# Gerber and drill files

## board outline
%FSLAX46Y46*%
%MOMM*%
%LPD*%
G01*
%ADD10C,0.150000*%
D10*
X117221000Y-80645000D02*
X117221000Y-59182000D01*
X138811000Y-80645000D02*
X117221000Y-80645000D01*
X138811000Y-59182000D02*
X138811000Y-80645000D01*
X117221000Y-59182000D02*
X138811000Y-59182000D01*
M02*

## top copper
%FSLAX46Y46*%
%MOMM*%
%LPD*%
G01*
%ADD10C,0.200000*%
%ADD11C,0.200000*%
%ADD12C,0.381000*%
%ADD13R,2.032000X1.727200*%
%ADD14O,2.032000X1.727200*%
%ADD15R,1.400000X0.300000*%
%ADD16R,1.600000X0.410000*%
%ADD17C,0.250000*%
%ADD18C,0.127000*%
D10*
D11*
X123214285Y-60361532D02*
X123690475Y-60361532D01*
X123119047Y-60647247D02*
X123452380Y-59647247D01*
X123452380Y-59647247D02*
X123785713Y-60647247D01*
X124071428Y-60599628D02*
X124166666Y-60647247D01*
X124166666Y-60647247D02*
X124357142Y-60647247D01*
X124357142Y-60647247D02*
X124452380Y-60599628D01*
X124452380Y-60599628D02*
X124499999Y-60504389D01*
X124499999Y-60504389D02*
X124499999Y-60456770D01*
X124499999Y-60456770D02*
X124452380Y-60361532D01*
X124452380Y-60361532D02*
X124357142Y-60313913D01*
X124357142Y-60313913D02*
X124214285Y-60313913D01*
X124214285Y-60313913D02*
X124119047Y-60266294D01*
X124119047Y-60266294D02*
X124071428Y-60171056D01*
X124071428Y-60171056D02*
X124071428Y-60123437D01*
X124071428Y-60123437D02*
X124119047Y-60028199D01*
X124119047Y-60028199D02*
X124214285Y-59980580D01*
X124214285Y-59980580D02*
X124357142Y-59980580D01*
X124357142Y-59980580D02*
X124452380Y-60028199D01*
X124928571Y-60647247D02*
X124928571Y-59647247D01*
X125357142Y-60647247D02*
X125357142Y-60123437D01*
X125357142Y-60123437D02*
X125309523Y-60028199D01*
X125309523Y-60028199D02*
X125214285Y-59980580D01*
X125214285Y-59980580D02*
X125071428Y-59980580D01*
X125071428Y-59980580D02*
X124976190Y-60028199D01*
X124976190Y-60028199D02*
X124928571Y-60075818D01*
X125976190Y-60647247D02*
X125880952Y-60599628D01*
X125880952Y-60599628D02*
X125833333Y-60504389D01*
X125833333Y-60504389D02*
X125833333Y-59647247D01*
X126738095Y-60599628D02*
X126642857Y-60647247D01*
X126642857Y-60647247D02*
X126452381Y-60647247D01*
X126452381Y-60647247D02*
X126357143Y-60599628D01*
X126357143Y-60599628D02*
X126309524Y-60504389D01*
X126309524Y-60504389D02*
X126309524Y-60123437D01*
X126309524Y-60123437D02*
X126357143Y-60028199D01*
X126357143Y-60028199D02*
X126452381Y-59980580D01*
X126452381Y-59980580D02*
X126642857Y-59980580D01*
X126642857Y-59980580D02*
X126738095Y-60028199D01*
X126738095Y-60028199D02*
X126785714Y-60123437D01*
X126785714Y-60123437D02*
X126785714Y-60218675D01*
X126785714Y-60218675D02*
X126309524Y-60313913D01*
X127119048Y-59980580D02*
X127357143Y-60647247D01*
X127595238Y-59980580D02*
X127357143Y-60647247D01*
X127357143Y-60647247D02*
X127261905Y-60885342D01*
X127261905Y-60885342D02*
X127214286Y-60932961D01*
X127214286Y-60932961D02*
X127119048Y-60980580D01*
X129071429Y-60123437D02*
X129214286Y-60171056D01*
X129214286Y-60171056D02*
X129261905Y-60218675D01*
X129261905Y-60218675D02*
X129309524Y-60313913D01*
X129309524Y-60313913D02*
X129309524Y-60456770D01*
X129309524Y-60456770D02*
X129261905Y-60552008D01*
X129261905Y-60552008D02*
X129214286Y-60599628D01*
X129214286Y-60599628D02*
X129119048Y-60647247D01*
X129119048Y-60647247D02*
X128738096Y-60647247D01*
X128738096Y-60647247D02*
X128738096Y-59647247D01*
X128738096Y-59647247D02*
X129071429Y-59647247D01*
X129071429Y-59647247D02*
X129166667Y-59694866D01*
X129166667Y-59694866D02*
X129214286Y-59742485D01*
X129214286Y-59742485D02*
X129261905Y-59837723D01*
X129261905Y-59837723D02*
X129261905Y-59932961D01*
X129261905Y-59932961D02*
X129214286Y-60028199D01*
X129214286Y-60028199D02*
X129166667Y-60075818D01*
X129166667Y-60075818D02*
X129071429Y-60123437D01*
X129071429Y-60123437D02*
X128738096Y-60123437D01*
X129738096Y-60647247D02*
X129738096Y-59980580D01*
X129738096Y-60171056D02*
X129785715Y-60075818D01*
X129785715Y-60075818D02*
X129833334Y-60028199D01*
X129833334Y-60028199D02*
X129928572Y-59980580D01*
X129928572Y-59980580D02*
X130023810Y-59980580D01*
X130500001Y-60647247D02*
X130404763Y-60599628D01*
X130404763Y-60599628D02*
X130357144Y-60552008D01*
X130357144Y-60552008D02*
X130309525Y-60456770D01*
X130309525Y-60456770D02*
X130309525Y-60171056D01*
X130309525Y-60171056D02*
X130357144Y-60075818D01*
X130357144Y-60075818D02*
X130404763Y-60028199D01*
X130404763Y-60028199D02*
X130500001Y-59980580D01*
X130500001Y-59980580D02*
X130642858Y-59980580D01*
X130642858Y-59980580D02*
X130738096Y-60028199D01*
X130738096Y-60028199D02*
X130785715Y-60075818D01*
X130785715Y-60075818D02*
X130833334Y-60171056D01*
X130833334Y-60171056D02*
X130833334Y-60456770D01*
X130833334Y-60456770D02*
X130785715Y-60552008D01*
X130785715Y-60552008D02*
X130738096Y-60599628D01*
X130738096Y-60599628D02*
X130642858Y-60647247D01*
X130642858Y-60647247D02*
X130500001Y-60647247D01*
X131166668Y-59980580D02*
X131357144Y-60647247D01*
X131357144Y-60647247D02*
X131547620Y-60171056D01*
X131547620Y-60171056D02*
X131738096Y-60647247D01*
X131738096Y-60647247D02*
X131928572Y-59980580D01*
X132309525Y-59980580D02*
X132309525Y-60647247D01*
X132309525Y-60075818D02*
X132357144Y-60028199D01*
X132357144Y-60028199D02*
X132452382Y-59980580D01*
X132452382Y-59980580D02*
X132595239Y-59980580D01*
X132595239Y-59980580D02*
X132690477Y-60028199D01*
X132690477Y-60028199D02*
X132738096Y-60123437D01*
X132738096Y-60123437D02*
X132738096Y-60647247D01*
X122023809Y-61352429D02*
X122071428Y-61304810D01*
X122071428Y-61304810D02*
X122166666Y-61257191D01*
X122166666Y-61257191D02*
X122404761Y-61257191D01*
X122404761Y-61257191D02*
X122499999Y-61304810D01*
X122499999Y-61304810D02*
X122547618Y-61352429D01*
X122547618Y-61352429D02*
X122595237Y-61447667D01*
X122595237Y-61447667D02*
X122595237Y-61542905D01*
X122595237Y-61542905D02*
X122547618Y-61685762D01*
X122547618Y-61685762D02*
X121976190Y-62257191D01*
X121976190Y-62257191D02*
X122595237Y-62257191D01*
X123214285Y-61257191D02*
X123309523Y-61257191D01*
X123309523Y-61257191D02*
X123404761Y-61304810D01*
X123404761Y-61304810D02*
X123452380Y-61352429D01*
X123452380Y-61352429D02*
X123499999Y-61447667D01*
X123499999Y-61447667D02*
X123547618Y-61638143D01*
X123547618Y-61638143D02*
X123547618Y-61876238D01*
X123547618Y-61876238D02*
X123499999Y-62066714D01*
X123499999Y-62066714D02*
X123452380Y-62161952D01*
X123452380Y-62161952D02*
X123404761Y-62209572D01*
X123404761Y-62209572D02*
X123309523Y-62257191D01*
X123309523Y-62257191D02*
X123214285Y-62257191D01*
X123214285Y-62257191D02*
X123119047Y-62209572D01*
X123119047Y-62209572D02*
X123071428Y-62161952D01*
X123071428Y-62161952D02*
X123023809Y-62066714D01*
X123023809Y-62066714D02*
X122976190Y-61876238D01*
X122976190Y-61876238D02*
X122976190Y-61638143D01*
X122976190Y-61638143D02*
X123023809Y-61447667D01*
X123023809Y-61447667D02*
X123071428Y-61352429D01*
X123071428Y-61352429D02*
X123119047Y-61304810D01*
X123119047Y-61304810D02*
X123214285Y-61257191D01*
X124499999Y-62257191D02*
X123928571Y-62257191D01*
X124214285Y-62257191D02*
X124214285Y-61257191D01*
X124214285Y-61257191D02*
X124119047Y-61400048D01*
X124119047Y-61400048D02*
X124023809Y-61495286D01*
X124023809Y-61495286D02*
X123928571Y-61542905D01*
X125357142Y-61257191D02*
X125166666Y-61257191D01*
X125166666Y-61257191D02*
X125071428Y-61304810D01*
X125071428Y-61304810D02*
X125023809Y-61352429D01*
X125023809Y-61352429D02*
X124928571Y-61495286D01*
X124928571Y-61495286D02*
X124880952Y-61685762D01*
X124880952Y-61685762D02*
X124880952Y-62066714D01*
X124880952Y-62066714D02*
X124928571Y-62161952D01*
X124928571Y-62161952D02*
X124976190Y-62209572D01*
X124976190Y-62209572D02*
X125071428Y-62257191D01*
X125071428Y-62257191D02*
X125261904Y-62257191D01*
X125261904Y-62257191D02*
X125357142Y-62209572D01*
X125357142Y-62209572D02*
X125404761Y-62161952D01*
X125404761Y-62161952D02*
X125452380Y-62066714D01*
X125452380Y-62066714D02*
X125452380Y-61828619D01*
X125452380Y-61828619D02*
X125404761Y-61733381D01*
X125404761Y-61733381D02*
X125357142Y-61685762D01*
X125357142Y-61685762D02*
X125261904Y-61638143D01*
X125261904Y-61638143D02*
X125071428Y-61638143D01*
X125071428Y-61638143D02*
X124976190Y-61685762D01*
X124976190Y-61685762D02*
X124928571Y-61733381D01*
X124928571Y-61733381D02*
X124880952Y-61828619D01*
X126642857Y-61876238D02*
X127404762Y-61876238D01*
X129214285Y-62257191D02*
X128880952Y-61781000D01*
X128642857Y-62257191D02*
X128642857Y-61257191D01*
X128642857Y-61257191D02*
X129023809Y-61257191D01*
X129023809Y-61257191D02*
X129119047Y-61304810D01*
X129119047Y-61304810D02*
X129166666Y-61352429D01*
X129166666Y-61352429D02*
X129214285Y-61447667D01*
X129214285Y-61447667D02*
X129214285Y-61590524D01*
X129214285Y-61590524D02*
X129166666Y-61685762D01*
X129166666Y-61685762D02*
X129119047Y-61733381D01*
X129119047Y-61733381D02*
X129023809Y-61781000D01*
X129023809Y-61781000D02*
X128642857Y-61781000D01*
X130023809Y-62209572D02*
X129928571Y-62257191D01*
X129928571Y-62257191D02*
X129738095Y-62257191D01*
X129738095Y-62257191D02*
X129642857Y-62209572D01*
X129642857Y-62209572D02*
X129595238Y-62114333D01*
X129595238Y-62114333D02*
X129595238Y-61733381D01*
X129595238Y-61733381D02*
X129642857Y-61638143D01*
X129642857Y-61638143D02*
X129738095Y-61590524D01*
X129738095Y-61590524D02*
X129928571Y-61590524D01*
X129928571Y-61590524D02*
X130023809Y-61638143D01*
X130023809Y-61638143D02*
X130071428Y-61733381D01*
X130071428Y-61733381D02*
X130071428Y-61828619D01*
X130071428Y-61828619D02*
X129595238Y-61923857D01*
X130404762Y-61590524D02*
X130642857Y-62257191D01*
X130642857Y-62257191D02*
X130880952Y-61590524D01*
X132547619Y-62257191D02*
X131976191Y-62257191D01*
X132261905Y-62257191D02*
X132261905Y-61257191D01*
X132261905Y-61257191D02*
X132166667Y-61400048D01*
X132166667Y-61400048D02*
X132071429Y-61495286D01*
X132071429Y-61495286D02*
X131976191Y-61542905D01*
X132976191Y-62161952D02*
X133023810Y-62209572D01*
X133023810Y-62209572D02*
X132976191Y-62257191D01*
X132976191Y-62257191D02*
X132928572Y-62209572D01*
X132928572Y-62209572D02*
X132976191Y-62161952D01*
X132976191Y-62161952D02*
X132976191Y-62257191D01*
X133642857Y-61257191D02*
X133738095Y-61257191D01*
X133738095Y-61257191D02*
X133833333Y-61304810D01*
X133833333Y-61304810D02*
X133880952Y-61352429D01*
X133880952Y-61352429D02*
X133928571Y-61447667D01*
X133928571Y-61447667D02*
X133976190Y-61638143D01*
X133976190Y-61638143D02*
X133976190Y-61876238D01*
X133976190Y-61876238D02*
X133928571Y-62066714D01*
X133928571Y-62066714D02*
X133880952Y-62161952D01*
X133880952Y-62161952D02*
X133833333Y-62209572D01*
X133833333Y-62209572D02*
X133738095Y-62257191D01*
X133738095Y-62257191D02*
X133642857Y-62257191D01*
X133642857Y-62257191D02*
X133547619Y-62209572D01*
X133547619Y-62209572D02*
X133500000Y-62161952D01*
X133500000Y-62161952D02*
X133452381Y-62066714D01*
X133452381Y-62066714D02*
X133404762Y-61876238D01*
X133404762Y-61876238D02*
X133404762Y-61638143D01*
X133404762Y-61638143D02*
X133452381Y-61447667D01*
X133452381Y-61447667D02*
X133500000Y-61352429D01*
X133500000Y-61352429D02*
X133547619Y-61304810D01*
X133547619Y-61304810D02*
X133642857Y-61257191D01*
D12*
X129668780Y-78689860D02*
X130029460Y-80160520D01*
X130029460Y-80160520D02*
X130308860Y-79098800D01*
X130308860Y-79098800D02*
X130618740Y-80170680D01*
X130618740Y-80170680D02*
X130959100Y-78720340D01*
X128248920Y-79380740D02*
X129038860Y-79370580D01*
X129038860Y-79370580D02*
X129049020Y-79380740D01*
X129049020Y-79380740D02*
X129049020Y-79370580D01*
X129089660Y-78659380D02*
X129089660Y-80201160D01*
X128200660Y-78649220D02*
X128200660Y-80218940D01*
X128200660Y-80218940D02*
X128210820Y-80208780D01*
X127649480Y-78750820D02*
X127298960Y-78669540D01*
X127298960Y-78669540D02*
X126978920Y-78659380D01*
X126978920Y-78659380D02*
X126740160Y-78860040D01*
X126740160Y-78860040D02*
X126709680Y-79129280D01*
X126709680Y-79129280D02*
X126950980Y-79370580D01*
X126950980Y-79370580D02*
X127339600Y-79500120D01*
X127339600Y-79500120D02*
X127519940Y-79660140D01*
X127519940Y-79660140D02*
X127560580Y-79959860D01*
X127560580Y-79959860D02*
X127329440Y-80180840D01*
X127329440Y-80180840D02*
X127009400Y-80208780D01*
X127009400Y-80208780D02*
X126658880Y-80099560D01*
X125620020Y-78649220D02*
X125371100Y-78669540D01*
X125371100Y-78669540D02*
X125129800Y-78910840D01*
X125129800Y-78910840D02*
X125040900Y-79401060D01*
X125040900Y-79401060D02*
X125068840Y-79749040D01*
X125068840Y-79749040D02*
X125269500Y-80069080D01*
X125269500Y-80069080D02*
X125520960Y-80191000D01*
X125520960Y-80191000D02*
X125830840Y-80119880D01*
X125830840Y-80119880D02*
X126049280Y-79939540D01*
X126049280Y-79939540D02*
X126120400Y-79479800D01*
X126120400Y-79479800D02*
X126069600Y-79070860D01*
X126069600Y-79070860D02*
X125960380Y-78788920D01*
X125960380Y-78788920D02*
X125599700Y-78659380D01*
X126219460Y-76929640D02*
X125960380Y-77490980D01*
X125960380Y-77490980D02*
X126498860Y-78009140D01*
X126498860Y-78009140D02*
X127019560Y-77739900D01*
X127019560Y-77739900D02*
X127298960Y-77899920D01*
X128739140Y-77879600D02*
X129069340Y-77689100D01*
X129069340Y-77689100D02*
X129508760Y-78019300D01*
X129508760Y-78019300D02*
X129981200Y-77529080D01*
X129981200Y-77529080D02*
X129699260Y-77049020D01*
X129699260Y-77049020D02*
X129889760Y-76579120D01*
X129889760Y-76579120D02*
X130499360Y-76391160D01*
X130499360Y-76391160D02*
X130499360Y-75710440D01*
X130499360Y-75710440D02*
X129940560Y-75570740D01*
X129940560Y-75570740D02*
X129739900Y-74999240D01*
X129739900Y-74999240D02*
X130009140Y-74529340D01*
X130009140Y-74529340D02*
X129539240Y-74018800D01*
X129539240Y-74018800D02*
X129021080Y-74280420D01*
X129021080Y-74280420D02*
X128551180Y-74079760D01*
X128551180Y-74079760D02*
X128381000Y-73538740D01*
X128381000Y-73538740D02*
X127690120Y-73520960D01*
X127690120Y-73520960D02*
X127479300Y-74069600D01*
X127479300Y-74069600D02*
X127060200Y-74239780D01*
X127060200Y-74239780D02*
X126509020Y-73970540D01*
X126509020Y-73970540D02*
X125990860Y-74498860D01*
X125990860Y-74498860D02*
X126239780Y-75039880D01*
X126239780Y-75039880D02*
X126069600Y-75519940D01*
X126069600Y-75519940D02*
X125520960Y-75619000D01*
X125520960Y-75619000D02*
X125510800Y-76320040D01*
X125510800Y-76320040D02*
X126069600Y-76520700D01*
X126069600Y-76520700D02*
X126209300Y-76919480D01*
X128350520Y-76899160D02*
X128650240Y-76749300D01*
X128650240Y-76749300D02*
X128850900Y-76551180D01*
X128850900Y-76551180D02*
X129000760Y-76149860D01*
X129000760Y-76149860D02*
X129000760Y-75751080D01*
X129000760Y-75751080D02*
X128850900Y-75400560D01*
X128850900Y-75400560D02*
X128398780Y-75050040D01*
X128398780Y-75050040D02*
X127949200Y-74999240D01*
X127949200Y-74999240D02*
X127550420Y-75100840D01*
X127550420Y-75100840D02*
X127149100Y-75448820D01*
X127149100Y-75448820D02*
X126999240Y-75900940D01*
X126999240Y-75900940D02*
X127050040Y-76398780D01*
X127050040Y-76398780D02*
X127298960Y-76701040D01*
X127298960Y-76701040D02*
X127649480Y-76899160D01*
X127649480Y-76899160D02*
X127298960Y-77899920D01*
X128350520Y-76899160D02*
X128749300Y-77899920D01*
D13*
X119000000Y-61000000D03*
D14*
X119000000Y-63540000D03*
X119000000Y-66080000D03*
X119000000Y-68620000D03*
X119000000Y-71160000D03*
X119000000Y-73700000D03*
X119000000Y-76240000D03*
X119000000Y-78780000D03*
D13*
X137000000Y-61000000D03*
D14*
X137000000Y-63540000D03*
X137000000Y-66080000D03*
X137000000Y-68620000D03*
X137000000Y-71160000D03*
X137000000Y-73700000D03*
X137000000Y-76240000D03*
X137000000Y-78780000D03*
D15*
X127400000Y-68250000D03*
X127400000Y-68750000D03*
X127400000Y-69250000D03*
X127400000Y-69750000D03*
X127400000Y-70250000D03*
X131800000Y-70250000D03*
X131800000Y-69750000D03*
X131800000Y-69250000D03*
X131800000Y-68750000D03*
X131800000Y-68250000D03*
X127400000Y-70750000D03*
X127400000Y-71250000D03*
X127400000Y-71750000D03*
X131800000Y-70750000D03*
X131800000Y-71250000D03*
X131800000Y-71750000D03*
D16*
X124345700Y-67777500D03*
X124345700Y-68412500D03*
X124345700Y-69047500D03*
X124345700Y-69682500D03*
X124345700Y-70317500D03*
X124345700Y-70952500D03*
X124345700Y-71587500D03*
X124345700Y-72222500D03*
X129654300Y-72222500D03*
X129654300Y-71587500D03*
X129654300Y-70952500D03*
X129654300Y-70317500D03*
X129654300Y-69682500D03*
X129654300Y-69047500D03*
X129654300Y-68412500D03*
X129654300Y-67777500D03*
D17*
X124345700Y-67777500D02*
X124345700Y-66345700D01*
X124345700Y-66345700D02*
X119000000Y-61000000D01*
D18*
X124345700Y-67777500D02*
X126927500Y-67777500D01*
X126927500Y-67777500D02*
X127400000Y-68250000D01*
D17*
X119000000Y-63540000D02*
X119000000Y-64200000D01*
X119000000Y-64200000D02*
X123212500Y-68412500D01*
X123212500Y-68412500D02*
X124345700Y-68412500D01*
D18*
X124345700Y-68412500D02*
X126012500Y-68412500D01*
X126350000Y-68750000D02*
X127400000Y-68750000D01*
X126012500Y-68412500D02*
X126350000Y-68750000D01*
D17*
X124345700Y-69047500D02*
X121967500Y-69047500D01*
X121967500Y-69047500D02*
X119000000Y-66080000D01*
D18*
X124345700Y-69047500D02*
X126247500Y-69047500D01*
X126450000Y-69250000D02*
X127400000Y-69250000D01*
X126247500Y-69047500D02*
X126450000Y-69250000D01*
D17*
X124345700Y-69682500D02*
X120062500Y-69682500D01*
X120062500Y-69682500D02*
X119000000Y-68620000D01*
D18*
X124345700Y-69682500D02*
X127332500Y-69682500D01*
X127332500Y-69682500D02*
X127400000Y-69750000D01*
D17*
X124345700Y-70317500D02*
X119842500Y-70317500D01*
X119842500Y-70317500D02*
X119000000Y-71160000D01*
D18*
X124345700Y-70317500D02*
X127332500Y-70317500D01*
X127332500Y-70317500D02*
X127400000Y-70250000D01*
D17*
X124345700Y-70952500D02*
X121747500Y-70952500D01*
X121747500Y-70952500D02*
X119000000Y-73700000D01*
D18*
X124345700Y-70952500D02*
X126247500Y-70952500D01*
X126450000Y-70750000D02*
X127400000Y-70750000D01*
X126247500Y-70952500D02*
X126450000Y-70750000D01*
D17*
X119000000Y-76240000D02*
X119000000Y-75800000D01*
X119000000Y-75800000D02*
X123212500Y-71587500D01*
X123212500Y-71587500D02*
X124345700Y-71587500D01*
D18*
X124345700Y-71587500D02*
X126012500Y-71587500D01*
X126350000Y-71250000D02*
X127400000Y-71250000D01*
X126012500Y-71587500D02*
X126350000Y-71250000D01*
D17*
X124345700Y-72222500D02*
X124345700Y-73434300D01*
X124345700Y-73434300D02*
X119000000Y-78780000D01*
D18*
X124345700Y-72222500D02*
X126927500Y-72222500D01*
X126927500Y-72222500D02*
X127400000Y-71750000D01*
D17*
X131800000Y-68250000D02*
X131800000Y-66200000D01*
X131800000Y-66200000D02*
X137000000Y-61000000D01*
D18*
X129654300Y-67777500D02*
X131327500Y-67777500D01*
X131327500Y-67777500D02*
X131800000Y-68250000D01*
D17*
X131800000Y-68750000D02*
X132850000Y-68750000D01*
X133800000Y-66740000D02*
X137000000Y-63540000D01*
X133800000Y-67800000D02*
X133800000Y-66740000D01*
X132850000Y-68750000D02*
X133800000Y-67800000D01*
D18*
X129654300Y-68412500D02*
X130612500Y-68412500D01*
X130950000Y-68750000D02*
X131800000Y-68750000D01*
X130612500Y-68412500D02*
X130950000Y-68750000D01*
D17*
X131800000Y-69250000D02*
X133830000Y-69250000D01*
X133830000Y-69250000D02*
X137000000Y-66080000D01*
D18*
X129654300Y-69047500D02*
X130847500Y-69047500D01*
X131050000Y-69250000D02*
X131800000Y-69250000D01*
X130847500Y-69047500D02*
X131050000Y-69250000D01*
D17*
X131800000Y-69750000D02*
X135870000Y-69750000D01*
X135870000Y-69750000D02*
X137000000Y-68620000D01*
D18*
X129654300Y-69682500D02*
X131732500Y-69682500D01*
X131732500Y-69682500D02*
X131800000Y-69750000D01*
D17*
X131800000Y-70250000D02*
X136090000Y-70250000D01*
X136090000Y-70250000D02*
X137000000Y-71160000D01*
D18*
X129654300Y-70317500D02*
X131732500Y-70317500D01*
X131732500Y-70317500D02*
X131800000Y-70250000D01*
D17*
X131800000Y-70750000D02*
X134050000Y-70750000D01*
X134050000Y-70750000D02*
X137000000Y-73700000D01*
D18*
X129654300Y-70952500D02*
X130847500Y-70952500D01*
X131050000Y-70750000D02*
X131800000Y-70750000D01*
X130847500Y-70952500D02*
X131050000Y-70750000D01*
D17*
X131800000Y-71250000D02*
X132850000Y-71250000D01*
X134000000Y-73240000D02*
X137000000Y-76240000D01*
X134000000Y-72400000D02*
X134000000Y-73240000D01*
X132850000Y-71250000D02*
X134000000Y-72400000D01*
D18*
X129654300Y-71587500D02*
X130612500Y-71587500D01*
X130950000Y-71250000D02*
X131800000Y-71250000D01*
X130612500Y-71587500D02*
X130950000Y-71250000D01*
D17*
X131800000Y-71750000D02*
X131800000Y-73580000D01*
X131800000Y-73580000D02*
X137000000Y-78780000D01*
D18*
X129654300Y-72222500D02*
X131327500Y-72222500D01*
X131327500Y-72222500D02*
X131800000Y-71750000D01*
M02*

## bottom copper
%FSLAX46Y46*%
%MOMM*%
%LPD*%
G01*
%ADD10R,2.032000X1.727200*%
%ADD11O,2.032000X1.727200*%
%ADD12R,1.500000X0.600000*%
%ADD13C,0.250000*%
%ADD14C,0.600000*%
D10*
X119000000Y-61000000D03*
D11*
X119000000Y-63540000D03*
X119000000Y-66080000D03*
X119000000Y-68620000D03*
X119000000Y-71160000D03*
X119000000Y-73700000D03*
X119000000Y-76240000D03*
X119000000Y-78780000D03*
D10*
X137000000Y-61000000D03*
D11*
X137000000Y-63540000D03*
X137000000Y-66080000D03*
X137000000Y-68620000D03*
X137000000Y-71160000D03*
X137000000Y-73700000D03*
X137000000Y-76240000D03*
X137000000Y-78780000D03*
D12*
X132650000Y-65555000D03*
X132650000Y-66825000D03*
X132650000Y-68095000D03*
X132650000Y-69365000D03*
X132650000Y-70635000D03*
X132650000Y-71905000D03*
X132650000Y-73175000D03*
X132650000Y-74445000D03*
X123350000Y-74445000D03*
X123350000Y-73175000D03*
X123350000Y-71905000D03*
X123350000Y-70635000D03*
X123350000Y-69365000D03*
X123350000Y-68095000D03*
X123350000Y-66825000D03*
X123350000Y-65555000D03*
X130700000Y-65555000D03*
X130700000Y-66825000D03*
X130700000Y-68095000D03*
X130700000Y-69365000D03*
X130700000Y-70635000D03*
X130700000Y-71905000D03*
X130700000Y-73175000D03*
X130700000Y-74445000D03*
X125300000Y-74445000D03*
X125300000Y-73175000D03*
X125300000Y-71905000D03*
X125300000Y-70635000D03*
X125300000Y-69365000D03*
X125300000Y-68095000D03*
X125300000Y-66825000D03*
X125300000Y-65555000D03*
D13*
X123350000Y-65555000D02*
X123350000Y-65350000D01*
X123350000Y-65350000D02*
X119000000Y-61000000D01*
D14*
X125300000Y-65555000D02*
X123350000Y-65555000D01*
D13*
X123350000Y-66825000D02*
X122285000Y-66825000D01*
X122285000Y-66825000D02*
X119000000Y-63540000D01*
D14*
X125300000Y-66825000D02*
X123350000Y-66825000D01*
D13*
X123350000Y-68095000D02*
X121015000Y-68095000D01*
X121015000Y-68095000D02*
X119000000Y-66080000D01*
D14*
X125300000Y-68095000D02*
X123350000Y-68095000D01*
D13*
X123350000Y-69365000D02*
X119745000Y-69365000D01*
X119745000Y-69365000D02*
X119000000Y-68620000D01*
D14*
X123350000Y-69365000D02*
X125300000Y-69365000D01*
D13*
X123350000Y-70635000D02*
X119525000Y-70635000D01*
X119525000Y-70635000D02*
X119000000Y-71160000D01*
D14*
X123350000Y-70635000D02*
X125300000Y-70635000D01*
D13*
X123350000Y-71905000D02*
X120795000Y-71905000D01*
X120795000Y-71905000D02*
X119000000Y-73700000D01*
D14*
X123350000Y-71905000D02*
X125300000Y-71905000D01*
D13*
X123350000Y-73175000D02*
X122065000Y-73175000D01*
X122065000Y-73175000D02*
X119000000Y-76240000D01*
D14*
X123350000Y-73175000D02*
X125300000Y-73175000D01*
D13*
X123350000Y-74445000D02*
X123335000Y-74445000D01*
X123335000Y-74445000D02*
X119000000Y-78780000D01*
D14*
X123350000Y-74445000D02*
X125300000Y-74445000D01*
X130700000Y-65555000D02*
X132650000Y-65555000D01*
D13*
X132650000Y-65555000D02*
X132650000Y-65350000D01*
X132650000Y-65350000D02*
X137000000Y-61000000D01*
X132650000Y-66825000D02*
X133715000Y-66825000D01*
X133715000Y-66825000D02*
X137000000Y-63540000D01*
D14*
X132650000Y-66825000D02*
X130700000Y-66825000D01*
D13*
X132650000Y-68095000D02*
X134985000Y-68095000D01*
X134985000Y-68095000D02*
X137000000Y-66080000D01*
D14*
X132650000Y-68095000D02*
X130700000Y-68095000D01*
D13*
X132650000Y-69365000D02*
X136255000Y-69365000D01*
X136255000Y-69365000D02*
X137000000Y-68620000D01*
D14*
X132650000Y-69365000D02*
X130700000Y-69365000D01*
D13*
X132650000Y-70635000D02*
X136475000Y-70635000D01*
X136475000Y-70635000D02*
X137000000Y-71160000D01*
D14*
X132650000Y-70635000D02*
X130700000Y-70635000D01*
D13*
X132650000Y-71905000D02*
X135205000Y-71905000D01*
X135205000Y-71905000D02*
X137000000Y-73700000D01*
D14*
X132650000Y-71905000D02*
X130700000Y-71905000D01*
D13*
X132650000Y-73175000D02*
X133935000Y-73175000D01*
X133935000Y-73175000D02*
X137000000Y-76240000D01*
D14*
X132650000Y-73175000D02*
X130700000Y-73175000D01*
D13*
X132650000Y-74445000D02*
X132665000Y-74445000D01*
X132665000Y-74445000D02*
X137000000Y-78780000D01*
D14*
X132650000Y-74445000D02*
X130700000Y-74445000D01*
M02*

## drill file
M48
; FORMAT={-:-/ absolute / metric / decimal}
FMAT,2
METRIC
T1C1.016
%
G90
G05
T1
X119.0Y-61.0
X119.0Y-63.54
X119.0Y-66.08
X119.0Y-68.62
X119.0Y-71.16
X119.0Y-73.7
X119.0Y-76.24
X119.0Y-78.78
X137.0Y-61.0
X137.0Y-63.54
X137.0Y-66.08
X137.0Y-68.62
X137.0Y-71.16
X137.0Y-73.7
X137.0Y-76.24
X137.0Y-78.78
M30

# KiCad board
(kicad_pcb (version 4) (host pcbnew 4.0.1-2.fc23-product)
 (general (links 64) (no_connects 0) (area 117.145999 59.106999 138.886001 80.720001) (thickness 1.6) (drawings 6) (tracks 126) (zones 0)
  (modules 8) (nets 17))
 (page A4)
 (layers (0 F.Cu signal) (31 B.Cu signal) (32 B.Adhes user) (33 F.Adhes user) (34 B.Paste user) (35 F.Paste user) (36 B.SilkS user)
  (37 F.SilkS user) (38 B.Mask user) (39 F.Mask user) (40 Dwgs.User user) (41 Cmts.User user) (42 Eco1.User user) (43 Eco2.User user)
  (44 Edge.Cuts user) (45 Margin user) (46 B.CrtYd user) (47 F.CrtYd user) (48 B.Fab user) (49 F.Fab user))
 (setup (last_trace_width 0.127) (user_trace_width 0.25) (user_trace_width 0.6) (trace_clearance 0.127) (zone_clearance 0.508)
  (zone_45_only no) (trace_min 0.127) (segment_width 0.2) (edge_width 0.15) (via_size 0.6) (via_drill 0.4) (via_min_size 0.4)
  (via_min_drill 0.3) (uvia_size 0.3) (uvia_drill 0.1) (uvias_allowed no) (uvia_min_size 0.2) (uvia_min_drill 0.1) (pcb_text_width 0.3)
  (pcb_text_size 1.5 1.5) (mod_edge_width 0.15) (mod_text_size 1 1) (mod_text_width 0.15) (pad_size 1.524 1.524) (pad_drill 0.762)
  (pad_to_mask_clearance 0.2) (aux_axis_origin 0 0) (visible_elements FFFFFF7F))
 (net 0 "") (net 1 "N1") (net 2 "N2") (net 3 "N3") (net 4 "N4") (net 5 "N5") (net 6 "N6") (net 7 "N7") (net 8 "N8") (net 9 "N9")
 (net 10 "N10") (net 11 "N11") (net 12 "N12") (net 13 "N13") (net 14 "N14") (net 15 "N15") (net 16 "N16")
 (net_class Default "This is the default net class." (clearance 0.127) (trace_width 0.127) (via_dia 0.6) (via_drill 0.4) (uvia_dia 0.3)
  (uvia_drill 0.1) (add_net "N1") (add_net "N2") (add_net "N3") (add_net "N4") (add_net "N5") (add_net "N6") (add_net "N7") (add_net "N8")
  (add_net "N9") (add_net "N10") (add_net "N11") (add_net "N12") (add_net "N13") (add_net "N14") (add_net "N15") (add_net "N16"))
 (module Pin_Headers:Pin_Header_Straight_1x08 (layer F.Cu) (at 119 61)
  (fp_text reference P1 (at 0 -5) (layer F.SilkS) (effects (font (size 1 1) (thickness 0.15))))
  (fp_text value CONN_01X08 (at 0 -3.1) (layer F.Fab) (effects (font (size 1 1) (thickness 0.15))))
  (pad 1 thru_hole rect (at 0 0) (size 2.032 1.7272) (drill 1.016) (layers *.Cu *.Mask F.SilkS) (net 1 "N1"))
  (pad 2 thru_hole oval (at 0 2.54) (size 2.032 1.7272) (drill 1.016) (layers *.Cu *.Mask F.SilkS) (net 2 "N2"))
  (pad 3 thru_hole oval (at 0 5.08) (size 2.032 1.7272) (drill 1.016) (layers *.Cu *.Mask F.SilkS) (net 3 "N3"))
  (pad 4 thru_hole oval (at 0 7.62) (size 2.032 1.7272) (drill 1.016) (layers *.Cu *.Mask F.SilkS) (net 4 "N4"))
  (pad 5 thru_hole oval (at 0 10.16) (size 2.032 1.7272) (drill 1.016) (layers *.Cu *.Mask F.SilkS) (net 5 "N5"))
  (pad 6 thru_hole oval (at 0 12.7) (size 2.032 1.7272) (drill 1.016) (layers *.Cu *.Mask F.SilkS) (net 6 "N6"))
  (pad 7 thru_hole oval (at 0 15.24) (size 2.032 1.7272) (drill 1.016) (layers *.Cu *.Mask F.SilkS) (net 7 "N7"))
  (pad 8 thru_hole oval (at 0 17.78) (size 2.032 1.7272) (drill 1.016) (layers *.Cu *.Mask F.SilkS) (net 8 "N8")))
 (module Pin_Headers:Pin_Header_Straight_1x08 (layer F.Cu) (at 137 61)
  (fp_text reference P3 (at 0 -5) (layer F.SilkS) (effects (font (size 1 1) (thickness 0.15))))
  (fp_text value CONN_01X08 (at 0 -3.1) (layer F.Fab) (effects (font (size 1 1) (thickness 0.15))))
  (pad 1 thru_hole rect (at 0 0) (size 2.032 1.7272) (drill 1.016) (layers *.Cu *.Mask F.SilkS) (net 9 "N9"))
  (pad 2 thru_hole oval (at 0 2.54) (size 2.032 1.7272) (drill 1.016) (layers *.Cu *.Mask F.SilkS) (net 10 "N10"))
  (pad 3 thru_hole oval (at 0 5.08) (size 2.032 1.7272) (drill 1.016) (layers *.Cu *.Mask F.SilkS) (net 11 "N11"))
  (pad 4 thru_hole oval (at 0 7.62) (size 2.032 1.7272) (drill 1.016) (layers *.Cu *.Mask F.SilkS) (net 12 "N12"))
  (pad 5 thru_hole oval (at 0 10.16) (size 2.032 1.7272) (drill 1.016) (layers *.Cu *.Mask F.SilkS) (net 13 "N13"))
  (pad 6 thru_hole oval (at 0 12.7) (size 2.032 1.7272) (drill 1.016) (layers *.Cu *.Mask F.SilkS) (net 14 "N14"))
  (pad 7 thru_hole oval (at 0 15.24) (size 2.032 1.7272) (drill 1.016) (layers *.Cu *.Mask F.SilkS) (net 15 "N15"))
  (pad 8 thru_hole oval (at 0 17.78) (size 2.032 1.7272) (drill 1.016) (layers *.Cu *.Mask F.SilkS) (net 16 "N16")))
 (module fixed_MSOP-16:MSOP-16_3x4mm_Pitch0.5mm (layer F.Cu) (at 129.6 70)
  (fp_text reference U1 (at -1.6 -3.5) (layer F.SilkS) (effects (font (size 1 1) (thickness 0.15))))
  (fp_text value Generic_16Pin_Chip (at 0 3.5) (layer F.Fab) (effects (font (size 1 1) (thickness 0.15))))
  (pad 1 smd rect (at -2.2 -1.75) (size 1.4 0.3) (layers F.Cu F.Paste F.Mask) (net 1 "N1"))
  (pad 2 smd rect (at -2.2 -1.25) (size 1.4 0.3) (layers F.Cu F.Paste F.Mask) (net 2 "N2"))
  (pad 3 smd rect (at -2.2 -0.75) (size 1.4 0.3) (layers F.Cu F.Paste F.Mask) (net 3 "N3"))
  (pad 4 smd rect (at -2.2 -0.25) (size 1.4 0.3) (layers F.Cu F.Paste F.Mask) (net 4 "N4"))
  (pad 5 smd rect (at -2.2 0.25) (size 1.4 0.3) (layers F.Cu F.Paste F.Mask) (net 5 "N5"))
  (pad 12 smd rect (at 2.2 0.25) (size 1.4 0.3) (layers F.Cu F.Paste F.Mask) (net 13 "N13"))
  (pad 13 smd rect (at 2.2 -0.25) (size 1.4 0.3) (layers F.Cu F.Paste F.Mask) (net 12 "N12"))
  (pad 14 smd rect (at 2.2 -0.75) (size 1.4 0.3) (layers F.Cu F.Paste F.Mask) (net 11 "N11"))
  (pad 15 smd rect (at 2.2 -1.25) (size 1.4 0.3) (layers F.Cu F.Paste F.Mask) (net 10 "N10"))
  (pad 16 smd rect (at 2.2 -1.75) (size 1.4 0.3) (layers F.Cu F.Paste F.Mask) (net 9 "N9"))
  (pad 6 smd rect (at -2.2 0.75) (size 1.4 0.3) (layers F.Cu F.Paste F.Mask) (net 6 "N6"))
  (pad 7 smd rect (at -2.2 1.25) (size 1.4 0.3) (layers F.Cu F.Paste F.Mask) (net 7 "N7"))
  (pad 8 smd rect (at -2.2 1.75) (size 1.4 0.3) (layers F.Cu F.Paste F.Mask) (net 8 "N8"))
  (pad 11 smd rect (at 2.2 0.75) (size 1.4 0.3) (layers F.Cu F.Paste F.Mask) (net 14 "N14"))
  (pad 10 smd rect (at 2.2 1.25) (size 1.4 0.3) (layers F.Cu F.Paste F.Mask) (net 15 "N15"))
  (pad 9 smd rect (at 2.2 1.75) (size 1.4 0.3) (layers F.Cu F.Paste F.Mask) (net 16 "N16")))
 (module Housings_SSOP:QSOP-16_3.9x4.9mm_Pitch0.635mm (layer F.Cu) (at 127 70)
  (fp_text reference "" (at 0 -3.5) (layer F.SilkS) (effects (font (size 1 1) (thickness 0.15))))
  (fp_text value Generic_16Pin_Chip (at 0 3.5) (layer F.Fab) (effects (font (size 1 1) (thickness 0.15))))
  (pad 1 smd rect (at -2.6543 -2.2225) (size 1.6 0.41) (layers F.Cu F.Paste F.Mask) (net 1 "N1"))
  (pad 2 smd rect (at -2.6543 -1.5875) (size 1.6 0.41) (layers F.Cu F.Paste F.Mask) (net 2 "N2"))
  (pad 3 smd rect (at -2.6543 -0.9525) (size 1.6 0.41) (layers F.Cu F.Paste F.Mask) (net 3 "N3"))
  (pad 4 smd rect (at -2.6543 -0.3175) (size 1.6 0.41) (layers F.Cu F.Paste F.Mask) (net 4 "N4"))
  (pad 5 smd rect (at -2.6543 0.3175) (size 1.6 0.41) (layers F.Cu F.Paste F.Mask) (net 5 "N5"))
  (pad 6 smd rect (at -2.6543 0.9525) (size 1.6 0.41) (layers F.Cu F.Paste F.Mask) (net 6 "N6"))
  (pad 7 smd rect (at -2.6543 1.5875) (size 1.6 0.41) (layers F.Cu F.Paste F.Mask) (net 7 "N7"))
  (pad 8 smd rect (at -2.6543 2.2225) (size 1.6 0.41) (layers F.Cu F.Paste F.Mask) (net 8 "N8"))
  (pad 9 smd rect (at 2.6543 2.2225) (size 1.6 0.41) (layers F.Cu F.Paste F.Mask) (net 16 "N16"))
  (pad 10 smd rect (at 2.6543 1.5875) (size 1.6 0.41) (layers F.Cu F.Paste F.Mask) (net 15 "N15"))
  (pad 11 smd rect (at 2.6543 0.9525) (size 1.6 0.41) (layers F.Cu F.Paste F.Mask) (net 14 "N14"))
  (pad 12 smd rect (at 2.6543 0.3175) (size 1.6 0.41) (layers F.Cu F.Paste F.Mask) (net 13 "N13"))
  (pad 13 smd rect (at 2.6543 -0.3175) (size 1.6 0.41) (layers F.Cu F.Paste F.Mask) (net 12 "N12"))
  (pad 14 smd rect (at 2.6543 -0.9525) (size 1.6 0.41) (layers F.Cu F.Paste F.Mask) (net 11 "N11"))
  (pad 15 smd rect (at 2.6543 -1.5875) (size 1.6 0.41) (layers F.Cu F.Paste F.Mask) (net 10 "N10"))
  (pad 16 smd rect (at 2.6543 -2.2225) (size 1.6 0.41) (layers F.Cu F.Paste F.Mask) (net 9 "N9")))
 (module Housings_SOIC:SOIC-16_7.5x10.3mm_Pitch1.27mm (layer B.Cu) (at 128 70 180)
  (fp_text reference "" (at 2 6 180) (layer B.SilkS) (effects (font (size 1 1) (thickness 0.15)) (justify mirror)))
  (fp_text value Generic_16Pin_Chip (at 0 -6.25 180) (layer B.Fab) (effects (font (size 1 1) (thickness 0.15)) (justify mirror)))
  (pad 1 smd rect (at -4.65 4.445 180) (size 1.5 0.6) (layers B.Cu B.Paste B.Mask) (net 9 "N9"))
  (pad 2 smd rect (at -4.65 3.175 180) (size 1.5 0.6) (layers B.Cu B.Paste B.Mask) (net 10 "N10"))
  (pad 3 smd rect (at -4.65 1.905 180) (size 1.5 0.6) (layers B.Cu B.Paste B.Mask) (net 11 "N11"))
  (pad 4 smd rect (at -4.65 0.635 180) (size 1.5 0.6) (layers B.Cu B.Paste B.Mask) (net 12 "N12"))
  (pad 5 smd rect (at -4.65 -0.635 180) (size 1.5 0.6) (layers B.Cu B.Paste B.Mask) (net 13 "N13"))
  (pad 6 smd rect (at -4.65 -1.905 180) (size 1.5 0.6) (layers B.Cu B.Paste B.Mask) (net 14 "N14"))
  (pad 7 smd rect (at -4.65 -3.175 180) (size 1.5 0.6) (layers B.Cu B.Paste B.Mask) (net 15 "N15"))
  (pad 8 smd rect (at -4.65 -4.445 180) (size 1.5 0.6) (layers B.Cu B.Paste B.Mask) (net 16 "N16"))
  (pad 9 smd rect (at 4.65 -4.445 180) (size 1.5 0.6) (layers B.Cu B.Paste B.Mask) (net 8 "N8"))
  (pad 10 smd rect (at 4.65 -3.175 180) (size 1.5 0.6) (layers B.Cu B.Paste B.Mask) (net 7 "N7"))
  (pad 11 smd rect (at 4.65 -1.905 180) (size 1.5 0.6) (layers B.Cu B.Paste B.Mask) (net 6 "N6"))
  (pad 12 smd rect (at 4.65 -0.635 180) (size 1.5 0.6) (layers B.Cu B.Paste B.Mask) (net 5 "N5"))
  (pad 13 smd rect (at 4.65 0.635 180) (size 1.5 0.6) (layers B.Cu B.Paste B.Mask) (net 4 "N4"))
  (pad 14 smd rect (at 4.65 1.905 180) (size 1.5 0.6) (layers B.Cu B.Paste B.Mask) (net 3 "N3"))
  (pad 15 smd rect (at 4.65 3.175 180) (size 1.5 0.6) (layers B.Cu B.Paste B.Mask) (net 2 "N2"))
  (pad 16 smd rect (at 4.65 4.445 180) (size 1.5 0.6) (layers B.Cu B.Paste B.Mask) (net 1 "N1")))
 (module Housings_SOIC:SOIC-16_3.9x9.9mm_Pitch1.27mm (layer B.Cu) (at 128 70 180)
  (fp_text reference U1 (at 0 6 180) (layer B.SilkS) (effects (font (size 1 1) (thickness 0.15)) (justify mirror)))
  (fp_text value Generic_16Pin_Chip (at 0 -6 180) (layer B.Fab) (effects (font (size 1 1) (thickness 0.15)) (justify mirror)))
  (pad 1 smd rect (at -2.7 4.445 180) (size 1.5 0.6) (layers B.Cu B.Paste B.Mask) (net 9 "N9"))
  (pad 2 smd rect (at -2.7 3.175 180) (size 1.5 0.6) (layers B.Cu B.Paste B.Mask) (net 10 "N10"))
  (pad 3 smd rect (at -2.7 1.905 180) (size 1.5 0.6) (layers B.Cu B.Paste B.Mask) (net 11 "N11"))
  (pad 4 smd rect (at -2.7 0.635 180) (size 1.5 0.6) (layers B.Cu B.Paste B.Mask) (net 12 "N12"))
  (pad 5 smd rect (at -2.7 -0.635 180) (size 1.5 0.6) (layers B.Cu B.Paste B.Mask) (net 13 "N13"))
  (pad 6 smd rect (at -2.7 -1.905 180) (size 1.5 0.6) (layers B.Cu B.Paste B.Mask) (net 14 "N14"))
  (pad 7 smd rect (at -2.7 -3.175 180) (size 1.5 0.6) (layers B.Cu B.Paste B.Mask) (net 15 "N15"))
  (pad 8 smd rect (at -2.7 -4.445 180) (size 1.5 0.6) (layers B.Cu B.Paste B.Mask) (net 16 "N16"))
  (pad 9 smd rect (at 2.7 -4.445 180) (size 1.5 0.6) (layers B.Cu B.Paste B.Mask) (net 8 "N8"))
  (pad 10 smd rect (at 2.7 -3.175 180) (size 1.5 0.6) (layers B.Cu B.Paste B.Mask) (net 7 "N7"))
  (pad 11 smd rect (at 2.7 -1.905 180) (size 1.5 0.6) (layers B.Cu B.Paste B.Mask) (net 6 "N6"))
  (pad 12 smd rect (at 2.7 -0.635 180) (size 1.5 0.6) (layers B.Cu B.Paste B.Mask) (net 5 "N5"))
  (pad 13 smd rect (at 2.7 0.635 180) (size 1.5 0.6) (layers B.Cu B.Paste B.Mask) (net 4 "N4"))
  (pad 14 smd rect (at 2.7 1.905 180) (size 1.5 0.6) (layers B.Cu B.Paste B.Mask) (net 3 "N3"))
  (pad 15 smd rect (at 2.7 3.175 180) (size 1.5 0.6) (layers B.Cu B.Paste B.Mask) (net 2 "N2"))
  (pad 16 smd rect (at 2.7 4.445 180) (size 1.5 0.6) (layers B.Cu B.Paste B.Mask) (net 1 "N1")))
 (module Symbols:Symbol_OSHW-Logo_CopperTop (layer F.Cu) (at 128 76)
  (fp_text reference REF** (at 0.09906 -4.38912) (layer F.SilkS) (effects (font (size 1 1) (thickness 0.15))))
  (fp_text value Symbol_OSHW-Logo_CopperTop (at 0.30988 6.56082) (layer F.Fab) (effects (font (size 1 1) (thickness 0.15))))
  (fp_line (start 1.66878 2.68986) (end 2.02946 4.16052) (layer F.Cu) (width 0.381))
  (fp_line (start 2.02946 4.16052) (end 2.30886 3.0988) (layer F.Cu) (width 0.381))
  (fp_line (start 2.30886 3.0988) (end 2.61874 4.17068) (layer F.Cu) (width 0.381))
  (fp_line (start 2.61874 4.17068) (end 2.9591 2.72034) (layer F.Cu) (width 0.381))
  (fp_line (start 0.24892 3.38074) (end 1.03886 3.37058) (layer F.Cu) (width 0.381))
  (fp_line (start 1.03886 3.37058) (end 1.04902 3.38074) (layer F.Cu) (width 0.381))
  (fp_line (start 1.04902 3.38074) (end 1.04902 3.37058) (layer F.Cu) (width 0.381))
  (fp_line (start 1.08966 2.65938) (end 1.08966 4.20116) (layer F.Cu) (width 0.381))
  (fp_line (start 0.20066 2.64922) (end 0.20066 4.21894) (layer F.Cu) (width 0.381))
  (fp_line (start 0.20066 4.21894) (end 0.21082 4.20878) (layer F.Cu) (width 0.381))
  (fp_line (start -0.35052 2.75082) (end -0.70104 2.66954) (layer F.Cu) (width 0.381))
  (fp_line (start -0.70104 2.66954) (end -1.02108 2.65938) (layer F.Cu) (width 0.381))
  (fp_line (start -1.02108 2.65938) (end -1.25984 2.86004) (layer F.Cu) (width 0.381))
  (fp_line (start -1.25984 2.86004) (end -1.29032 3.12928) (layer F.Cu) (width 0.381))
  (fp_line (start -1.29032 3.12928) (end -1.04902 3.37058) (layer F.Cu) (width 0.381))
  (fp_line (start -1.04902 3.37058) (end -0.6604 3.50012) (layer F.Cu) (width 0.381))
  (fp_line (start -0.6604 3.50012) (end -0.48006 3.66014) (layer F.Cu) (width 0.381))
  (fp_line (start -0.48006 3.66014) (end -0.43942 3.95986) (layer F.Cu) (width 0.381))
  (fp_line (start -0.43942 3.95986) (end -0.67056 4.18084) (layer F.Cu) (width 0.381))
  (fp_line (start -0.67056 4.18084) (end -0.9906 4.20878) (layer F.Cu) (width 0.381))
  (fp_line (start -0.9906 4.20878) (end -1.34112 4.09956) (layer F.Cu) (width 0.381))
  (fp_line (start -2.37998 2.64922) (end -2.6289 2.66954) (layer F.Cu) (width 0.381))
  (fp_line (start -2.6289 2.66954) (end -2.8702 2.91084) (layer F.Cu) (width 0.381))
  (fp_line (start -2.8702 2.91084) (end -2.9591 3.40106) (layer F.Cu) (width 0.381))
  (fp_line (start -2.9591 3.40106) (end -2.93116 3.74904) (layer F.Cu) (width 0.381))
  (fp_line (start -2.93116 3.74904) (end -2.7305 4.06908) (layer F.Cu) (width 0.381))
  (fp_line (start -2.7305 4.06908) (end -2.47904 4.191) (layer F.Cu) (width 0.381))
  (fp_line (start -2.47904 4.191) (end -2.16916 4.11988) (layer F.Cu) (width 0.381))
  (fp_line (start -2.16916 4.11988) (end -1.95072 3.93954) (layer F.Cu) (width 0.381))
  (fp_line (start -1.95072 3.93954) (end -1.8796 3.4798) (layer F.Cu) (width 0.381))
  (fp_line (start -1.8796 3.4798) (end -1.9304 3.07086) (layer F.Cu) (width 0.381))
  (fp_line (start -1.9304 3.07086) (end -2.03962 2.78892) (layer F.Cu) (width 0.381))
  (fp_line (start -2.03962 2.78892) (end -2.4003 2.65938) (layer F.Cu) (width 0.381))
  (fp_line (start -1.78054 0.92964) (end -2.03962 1.49098) (layer F.Cu) (width 0.381))
  (fp_line (start -2.03962 1.49098) (end -1.50114 2.00914) (layer F.Cu) (width 0.381))
  (fp_line (start -1.50114 2.00914) (end -0.98044 1.7399) (layer F.Cu) (width 0.381))
  (fp_line (start -0.98044 1.7399) (end -0.70104 1.89992) (layer F.Cu) (width 0.381))
  (fp_line (start 0.73914 1.8796) (end 1.06934 1.6891) (layer F.Cu) (width 0.381))
  (fp_line (start 1.06934 1.6891) (end 1.50876 2.0193) (layer F.Cu) (width 0.381))
  (fp_line (start 1.50876 2.0193) (end 1.9812 1.52908) (layer F.Cu) (width 0.381))
  (fp_line (start 1.9812 1.52908) (end 1.69926 1.04902) (layer F.Cu) (width 0.381))
  (fp_line (start 1.69926 1.04902) (end 1.88976 0.57912) (layer F.Cu) (width 0.381))
  (fp_line (start 1.88976 0.57912) (end 2.49936 0.39116) (layer F.Cu) (width 0.381))
  (fp_line (start 2.49936 0.39116) (end 2.49936 -0.28956) (layer F.Cu) (width 0.381))
  (fp_line (start 2.49936 -0.28956) (end 1.94056 -0.42926) (layer F.Cu) (width 0.381))
  (fp_line (start 1.94056 -0.42926) (end 1.7399 -1.00076) (layer F.Cu) (width 0.381))
  (fp_line (start 1.7399 -1.00076) (end 2.00914 -1.47066) (layer F.Cu) (width 0.381))
  (fp_line (start 2.00914 -1.47066) (end 1.53924 -1.9812) (layer F.Cu) (width 0.381))
  (fp_line (start 1.53924 -1.9812) (end 1.02108 -1.71958) (layer F.Cu) (width 0.381))
  (fp_line (start 1.02108 -1.71958) (end 0.55118 -1.92024) (layer F.Cu) (width 0.381))
  (fp_line (start 0.55118 -1.92024) (end 0.381 -2.46126) (layer F.Cu) (width 0.381))
  (fp_line (start 0.381 -2.46126) (end -0.30988 -2.47904) (layer F.Cu) (width 0.381))
  (fp_line (start -0.30988 -2.47904) (end -0.5207 -1.9304) (layer F.Cu) (width 0.381))
  (fp_line (start -0.5207 -1.9304) (end -0.9398 -1.76022) (layer F.Cu) (width 0.381))
  (fp_line (start -0.9398 -1.76022) (end -1.49098 -2.02946) (layer F.Cu) (width 0.381))
  (fp_line (start -1.49098 -2.02946) (end -2.00914 -1.50114) (layer F.Cu) (width 0.381))
  (fp_line (start -2.00914 -1.50114) (end -1.76022 -0.96012) (layer F.Cu) (width 0.381))
  (fp_line (start -1.76022 -0.96012) (end -1.9304 -0.48006) (layer F.Cu) (width 0.381))
  (fp_line (start -1.9304 -0.48006) (end -2.47904 -0.381) (layer F.Cu) (width 0.381))
  (fp_line (start -2.47904 -0.381) (end -2.4892 0.32004) (layer F.Cu) (width 0.381))
  (fp_line (start -2.4892 0.32004) (end -1.9304 0.5207) (layer F.Cu) (width 0.381))
  (fp_line (start -1.9304 0.5207) (end -1.7907 0.91948) (layer F.Cu) (width 0.381))
  (fp_line (start 0.35052 0.89916) (end 0.65024 0.7493) (layer F.Cu) (width 0.381))
  (fp_line (start 0.65024 0.7493) (end 0.8509 0.55118) (layer F.Cu) (width 0.381))
  (fp_line (start 0.8509 0.55118) (end 1.00076 0.14986) (layer F.Cu) (width 0.381))
  (fp_line (start 1.00076 0.14986) (end 1.00076 -0.24892) (layer F.Cu) (width 0.381))
  (fp_line (start 1.00076 -0.24892) (end 0.8509 -0.59944) (layer F.Cu) (width 0.381))
  (fp_line (start 0.8509 -0.59944) (end 0.39878 -0.94996) (layer F.Cu) (width 0.381))
  (fp_line (start 0.39878 -0.94996) (end -0.0508 -1.00076) (layer F.Cu) (width 0.381))
  (fp_line (start -0.0508 -1.00076) (end -0.44958 -0.89916) (layer F.Cu) (width 0.381))
  (fp_line (start -0.44958 -0.89916) (end -0.8509 -0.55118) (layer F.Cu) (width 0.381))
  (fp_line (start -0.8509 -0.55118) (end -1.00076 -0.09906) (layer F.Cu) (width 0.381))
  (fp_line (start -1.00076 -0.09906) (end -0.94996 0.39878) (layer F.Cu) (width 0.381))
  (fp_line (start -0.94996 0.39878) (end -0.70104 0.70104) (layer F.Cu) (width 0.381))
  (fp_line (start -0.70104 0.70104) (end -0.35052 0.89916) (layer F.Cu) (width 0.381))
  (fp_line (start -0.35052 0.89916) (end -0.70104 1.89992) (layer F.Cu) (width 0.381))
  (fp_line (start 0.35052 0.89916) (end 0.7493 1.89992) (layer F.Cu) (width 0.381)))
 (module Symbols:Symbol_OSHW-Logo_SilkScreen (layer F.Cu) (at 128 76)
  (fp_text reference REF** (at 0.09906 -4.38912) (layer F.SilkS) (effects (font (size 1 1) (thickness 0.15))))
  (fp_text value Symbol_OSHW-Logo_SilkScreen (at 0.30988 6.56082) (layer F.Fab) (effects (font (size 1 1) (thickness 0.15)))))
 (gr_line (start 117.221 80.645) (end 117.221 59.182) (angle 90) (layer Edge.Cuts) (width 0.15))
 (gr_line (start 138.811 80.645) (end 117.221 80.645) (angle 90) (layer Edge.Cuts) (width 0.15))
 (gr_line (start 138.811 59.182) (end 138.811 80.645) (angle 90) (layer Edge.Cuts) (width 0.15))
 (gr_line (start 117.221 59.182) (end 138.811 59.182) (angle 90) (layer Edge.Cuts) (width 0.15))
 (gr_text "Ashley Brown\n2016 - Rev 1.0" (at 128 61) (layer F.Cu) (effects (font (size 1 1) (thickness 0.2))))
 (segment (start 124.3457 67.7775) (end 124.3457 66.3457) (width 0.25) (layer F.Cu) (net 1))
 (segment (start 124.3457 66.3457) (end 119 61) (width 0.25) (layer F.Cu) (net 1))
 (segment (start 123.35 65.555) (end 123.35 65.35) (width 0.25) (layer B.Cu) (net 1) (status 30))
 (segment (start 123.35 65.35) (end 119 61) (width 0.25) (layer B.Cu) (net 1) (status 10))
 (segment (start 125.3 65.555) (end 123.35 65.555) (width 0.6) (layer B.Cu) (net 1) (status 20))
 (segment (start 124.3457 67.7775) (end 126.9275 67.7775) (width 0.127) (layer F.Cu) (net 1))
 (segment (start 126.9275 67.7775) (end 127.4 68.25) (width 0.127) (layer F.Cu) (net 1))
 (segment (start 119 63.54) (end 119 64.2) (width 0.25) (layer F.Cu) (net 2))
 (segment (start 119 64.2) (end 123.2125 68.4125) (width 0.25) (layer F.Cu) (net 2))
 (segment (start 123.2125 68.4125) (end 124.3457 68.4125) (width 0.25) (layer F.Cu) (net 2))
 (segment (start 123.35 66.825) (end 122.285 66.825) (width 0.25) (layer B.Cu) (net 2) (status 10))
 (segment (start 122.285 66.825) (end 119 63.54) (width 0.25) (layer B.Cu) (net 2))
 (segment (start 125.3 66.825) (end 123.35 66.825) (width 0.6) (layer B.Cu) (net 2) (status 20))
 (segment (start 124.3457 68.4125) (end 126.0125 68.4125) (width 0.127) (layer F.Cu) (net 2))
 (segment (start 126.35 68.75) (end 127.4 68.75) (width 0.127) (layer F.Cu) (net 2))
 (segment (start 126.0125 68.4125) (end 126.35 68.75) (width 0.127) (layer F.Cu) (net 2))
 (segment (start 124.3457 69.0475) (end 121.9675 69.0475) (width 0.25) (layer F.Cu) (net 3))
 (segment (start 121.9675 69.0475) (end 119 66.08) (width 0.25) (layer F.Cu) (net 3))
 (segment (start 123.35 68.095) (end 121.015 68.095) (width 0.25) (layer B.Cu) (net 3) (status 10))
 (segment (start 121.015 68.095) (end 119 66.08) (width 0.25) (layer B.Cu) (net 3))
 (segment (start 125.3 68.095) (end 123.35 68.095) (width 0.6) (layer B.Cu) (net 3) (status 20))
 (segment (start 124.3457 69.0475) (end 126.2475 69.0475) (width 0.127) (layer F.Cu) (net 3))
 (segment (start 126.45 69.25) (end 127.4 69.25) (width 0.127) (layer F.Cu) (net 3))
 (segment (start 126.2475 69.0475) (end 126.45 69.25) (width 0.127) (layer F.Cu) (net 3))
 (segment (start 124.3457 69.6825) (end 120.0625 69.6825) (width 0.25) (layer F.Cu) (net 4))
 (segment (start 120.0625 69.6825) (end 119 68.62) (width 0.25) (layer F.Cu) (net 4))
 (segment (start 123.35 69.365) (end 119.745 69.365) (width 0.25) (layer B.Cu) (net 4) (status 10))
 (segment (start 119.745 69.365) (end 119 68.62) (width 0.25) (layer B.Cu) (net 4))
 (segment (start 123.35 69.365) (end 125.3 69.365) (width 0.6) (layer B.Cu) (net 4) (status 10))
 (segment (start 124.3457 69.6825) (end 127.3325 69.6825) (width 0.127) (layer F.Cu) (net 4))
 (segment (start 127.3325 69.6825) (end 127.4 69.75) (width 0.127) (layer F.Cu) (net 4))
 (segment (start 124.3457 70.3175) (end 119.8425 70.3175) (width 0.25) (layer F.Cu) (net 5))
 (segment (start 119.8425 70.3175) (end 119 71.16) (width 0.25) (layer F.Cu) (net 5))
 (segment (start 123.35 70.635) (end 119.525 70.635) (width 0.25) (layer B.Cu) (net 5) (status 10))
 (segment (start 119.525 70.635) (end 119 71.16) (width 0.25) (layer B.Cu) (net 5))
 (segment (start 123.35 70.635) (end 125.3 70.635) (width 0.6) (layer B.Cu) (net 5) (status 10))
 (segment (start 124.3457 70.3175) (end 127.3325 70.3175) (width 0.127) (layer F.Cu) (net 5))
 (segment (start 127.3325 70.3175) (end 127.4 70.25) (width 0.127) (layer F.Cu) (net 5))
 (segment (start 124.3457 70.9525) (end 121.7475 70.9525) (width 0.25) (layer F.Cu) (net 6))
 (segment (start 121.7475 70.9525) (end 119 73.7) (width 0.25) (layer F.Cu) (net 6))
 (segment (start 123.35 71.905) (end 120.795 71.905) (width 0.25) (layer B.Cu) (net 6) (status 10))
 (segment (start 120.795 71.905) (end 119 73.7) (width 0.25) (layer B.Cu) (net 6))
 (segment (start 123.35 71.905) (end 125.3 71.905) (width 0.6) (layer B.Cu) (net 6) (status 10))
 (segment (start 124.3457 70.9525) (end 126.2475 70.9525) (width 0.127) (layer F.Cu) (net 6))
 (segment (start 126.45 70.75) (end 127.4 70.75) (width 0.127) (layer F.Cu) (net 6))
 (segment (start 126.2475 70.9525) (end 126.45 70.75) (width 0.127) (layer F.Cu) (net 6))
 (segment (start 119 76.24) (end 119 75.8) (width 0.25) (layer F.Cu) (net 7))
 (segment (start 119 75.8) (end 123.2125 71.5875) (width 0.25) (layer F.Cu) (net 7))
 (segment (start 123.2125 71.5875) (end 124.3457 71.5875) (width 0.25) (layer F.Cu) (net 7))
 (segment (start 123.35 73.175) (end 122.065 73.175) (width 0.25) (layer B.Cu) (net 7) (status 10))
 (segment (start 122.065 73.175) (end 119 76.24) (width 0.25) (layer B.Cu) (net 7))
 (segment (start 123.35 73.175) (end 125.3 73.175) (width 0.6) (layer B.Cu) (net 7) (status 10))
 (segment (start 124.3457 71.5875) (end 126.0125 71.5875) (width 0.127) (layer F.Cu) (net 7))
 (segment (start 126.35 71.25) (end 127.4 71.25) (width 0.127) (layer F.Cu) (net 7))
 (segment (start 126.0125 71.5875) (end 126.35 71.25) (width 0.127) (layer F.Cu) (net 7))
 (segment (start 124.3457 72.2225) (end 124.3457 73.4343) (width 0.25) (layer F.Cu) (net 8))
 (segment (start 124.3457 73.4343) (end 119 78.78) (width 0.25) (layer F.Cu) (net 8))
 (segment (start 123.35 74.445) (end 123.335 74.445) (width 0.25) (layer B.Cu) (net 8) (status 30))
 (segment (start 123.335 74.445) (end 119 78.78) (width 0.25) (layer B.Cu) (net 8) (status 10))
 (segment (start 123.35 74.445) (end 125.3 74.445) (width 0.6) (layer B.Cu) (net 8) (status 10))
 (segment (start 124.3457 72.2225) (end 126.9275 72.2225) (width 0.127) (layer F.Cu) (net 8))
 (segment (start 126.9275 72.2225) (end 127.4 71.75) (width 0.127) (layer F.Cu) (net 8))
 (segment (start 130.7 65.555) (end 132.65 65.555) (width 0.6) (layer B.Cu) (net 9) (status 20))
 (segment (start 131.8 68.25) (end 131.8 66.2) (width 0.25) (layer F.Cu) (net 9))
 (segment (start 131.8 66.2) (end 137 61) (width 0.25) (layer F.Cu) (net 9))
 (segment (start 132.65 65.555) (end 132.65 65.35) (width 0.25) (layer B.Cu) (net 9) (status 30))
 (segment (start 132.65 65.35) (end 137 61) (width 0.25) (layer B.Cu) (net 9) (status 10))
 (segment (start 129.6543 67.7775) (end 131.3275 67.7775) (width 0.127) (layer F.Cu) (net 9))
 (segment (start 131.3275 67.7775) (end 131.8 68.25) (width 0.127) (layer F.Cu) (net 9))
 (segment (start 131.8 68.75) (end 132.85 68.75) (width 0.25) (layer F.Cu) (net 10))
 (segment (start 133.8 66.74) (end 137 63.54) (width 0.25) (layer F.Cu) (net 10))
 (segment (start 133.8 67.8) (end 133.8 66.74) (width 0.25) (layer F.Cu) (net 10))
 (segment (start 132.85 68.75) (end 133.8 67.8) (width 0.25) (layer F.Cu) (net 10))
 (segment (start 132.65 66.825) (end 133.715 66.825) (width 0.25) (layer B.Cu) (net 10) (status 10))
 (segment (start 133.715 66.825) (end 137 63.54) (width 0.25) (layer B.Cu) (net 10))
 (segment (start 132.65 66.825) (end 130.7 66.825) (width 0.6) (layer B.Cu) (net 10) (status 10))
 (segment (start 129.6543 68.4125) (end 130.6125 68.4125) (width 0.127) (layer F.Cu) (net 10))
 (segment (start 130.95 68.75) (end 131.8 68.75) (width 0.127) (layer F.Cu) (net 10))
 (segment (start 130.6125 68.4125) (end 130.95 68.75) (width 0.127) (layer F.Cu) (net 10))
 (segment (start 131.8 69.25) (end 133.83 69.25) (width 0.25) (layer F.Cu) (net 11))
 (segment (start 133.83 69.25) (end 137 66.08) (width 0.25) (layer F.Cu) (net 11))
 (segment (start 132.65 68.095) (end 134.985 68.095) (width 0.25) (layer B.Cu) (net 11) (status 10))
 (segment (start 134.985 68.095) (end 137 66.08) (width 0.25) (layer B.Cu) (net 11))
 (segment (start 132.65 68.095) (end 130.7 68.095) (width 0.6) (layer B.Cu) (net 11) (status 10))
 (segment (start 129.6543 69.0475) (end 130.8475 69.0475) (width 0.127) (layer F.Cu) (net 11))
 (segment (start 131.05 69.25) (end 131.8 69.25) (width 0.127) (layer F.Cu) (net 11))
 (segment (start 130.8475 69.0475) (end 131.05 69.25) (width 0.127) (layer F.Cu) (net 11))
 (segment (start 131.8 69.75) (end 135.87 69.75) (width 0.25) (layer F.Cu) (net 12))
 (segment (start 135.87 69.75) (end 137 68.62) (width 0.25) (layer F.Cu) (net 12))
 (segment (start 132.65 69.365) (end 136.255 69.365) (width 0.25) (layer B.Cu) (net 12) (status 10))
 (segment (start 136.255 69.365) (end 137 68.62) (width 0.25) (layer B.Cu) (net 12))
 (segment (start 132.65 69.365) (end 130.7 69.365) (width 0.6) (layer B.Cu) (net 12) (status 10))
 (segment (start 129.6543 69.6825) (end 131.7325 69.6825) (width 0.127) (layer F.Cu) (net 12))
 (segment (start 131.7325 69.6825) (end 131.8 69.75) (width 0.127) (layer F.Cu) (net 12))
 (segment (start 131.8 70.25) (end 136.09 70.25) (width 0.25) (layer F.Cu) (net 13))
 (segment (start 136.09 70.25) (end 137 71.16) (width 0.25) (layer F.Cu) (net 13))
 (segment (start 132.65 70.635) (end 136.475 70.635) (width 0.25) (layer B.Cu) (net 13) (status 10))
 (segment (start 136.475 70.635) (end 137 71.16) (width 0.25) (layer B.Cu) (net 13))
 (segment (start 132.65 70.635) (end 130.7 70.635) (width 0.6) (layer B.Cu) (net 13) (status 10))
 (segment (start 129.6543 70.3175) (end 131.7325 70.3175) (width 0.127) (layer F.Cu) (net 13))
 (segment (start 131.7325 70.3175) (end 131.8 70.25) (width 0.127) (layer F.Cu) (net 13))
 (segment (start 131.8 70.75) (end 134.05 70.75) (width 0.25) (layer F.Cu) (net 14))
 (segment (start 134.05 70.75) (end 137 73.7) (width 0.25) (layer F.Cu) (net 14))
 (segment (start 132.65 71.905) (end 135.205 71.905) (width 0.25) (layer B.Cu) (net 14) (status 10))
 (segment (start 135.205 71.905) (end 137 73.7) (width 0.25) (layer B.Cu) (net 14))
 (segment (start 132.65 71.905) (end 130.7 71.905) (width 0.6) (layer B.Cu) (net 14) (status 10))
 (segment (start 129.6543 70.9525) (end 130.8475 70.9525) (width 0.127) (layer F.Cu) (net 14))
 (segment (start 131.05 70.75) (end 131.8 70.75) (width 0.127) (layer F.Cu) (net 14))
 (segment (start 130.8475 70.9525) (end 131.05 70.75) (width 0.127) (layer F.Cu) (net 14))
 (segment (start 131.8 71.25) (end 132.85 71.25) (width 0.25) (layer F.Cu) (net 15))
 (segment (start 134 73.24) (end 137 76.24) (width 0.25) (layer F.Cu) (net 15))
 (segment (start 134 72.4) (end 134 73.24) (width 0.25) (layer F.Cu) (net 15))
 (segment (start 132.85 71.25) (end 134 72.4) (width 0.25) (layer F.Cu) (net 15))
 (segment (start 132.65 73.175) (end 133.935 73.175) (width 0.25) (layer B.Cu) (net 15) (status 10))
 (segment (start 133.935 73.175) (end 137 76.24) (width 0.25) (layer B.Cu) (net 15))
 (segment (start 132.65 73.175) (end 130.7 73.175) (width 0.6) (layer B.Cu) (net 15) (status 10))
 (segment (start 129.6543 71.5875) (end 130.6125 71.5875) (width 0.127) (layer F.Cu) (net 15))
 (segment (start 130.95 71.25) (end 131.8 71.25) (width 0.127) (layer F.Cu) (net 15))
 (segment (start 130.6125 71.5875) (end 130.95 71.25) (width 0.127) (layer F.Cu) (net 15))
 (segment (start 131.8 71.75) (end 131.8 73.58) (width 0.25) (layer F.Cu) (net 16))
 (segment (start 131.8 73.58) (end 137 78.78) (width 0.25) (layer F.Cu) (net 16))
 (segment (start 132.65 74.445) (end 132.665 74.445) (width 0.25) (layer B.Cu) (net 16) (status 30))
 (segment (start 132.665 74.445) (end 137 78.78) (width 0.25) (layer B.Cu) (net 16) (status 10))
 (segment (start 132.65 74.445) (end 130.7 74.445) (width 0.6) (layer B.Cu) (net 16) (status 10))
 (segment (start 129.6543 72.2225) (end 131.3275 72.2225) (width 0.127) (layer F.Cu) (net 16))
 (segment (start 131.3275 72.2225) (end 131.8 71.75) (width 0.127) (layer F.Cu) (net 16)))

